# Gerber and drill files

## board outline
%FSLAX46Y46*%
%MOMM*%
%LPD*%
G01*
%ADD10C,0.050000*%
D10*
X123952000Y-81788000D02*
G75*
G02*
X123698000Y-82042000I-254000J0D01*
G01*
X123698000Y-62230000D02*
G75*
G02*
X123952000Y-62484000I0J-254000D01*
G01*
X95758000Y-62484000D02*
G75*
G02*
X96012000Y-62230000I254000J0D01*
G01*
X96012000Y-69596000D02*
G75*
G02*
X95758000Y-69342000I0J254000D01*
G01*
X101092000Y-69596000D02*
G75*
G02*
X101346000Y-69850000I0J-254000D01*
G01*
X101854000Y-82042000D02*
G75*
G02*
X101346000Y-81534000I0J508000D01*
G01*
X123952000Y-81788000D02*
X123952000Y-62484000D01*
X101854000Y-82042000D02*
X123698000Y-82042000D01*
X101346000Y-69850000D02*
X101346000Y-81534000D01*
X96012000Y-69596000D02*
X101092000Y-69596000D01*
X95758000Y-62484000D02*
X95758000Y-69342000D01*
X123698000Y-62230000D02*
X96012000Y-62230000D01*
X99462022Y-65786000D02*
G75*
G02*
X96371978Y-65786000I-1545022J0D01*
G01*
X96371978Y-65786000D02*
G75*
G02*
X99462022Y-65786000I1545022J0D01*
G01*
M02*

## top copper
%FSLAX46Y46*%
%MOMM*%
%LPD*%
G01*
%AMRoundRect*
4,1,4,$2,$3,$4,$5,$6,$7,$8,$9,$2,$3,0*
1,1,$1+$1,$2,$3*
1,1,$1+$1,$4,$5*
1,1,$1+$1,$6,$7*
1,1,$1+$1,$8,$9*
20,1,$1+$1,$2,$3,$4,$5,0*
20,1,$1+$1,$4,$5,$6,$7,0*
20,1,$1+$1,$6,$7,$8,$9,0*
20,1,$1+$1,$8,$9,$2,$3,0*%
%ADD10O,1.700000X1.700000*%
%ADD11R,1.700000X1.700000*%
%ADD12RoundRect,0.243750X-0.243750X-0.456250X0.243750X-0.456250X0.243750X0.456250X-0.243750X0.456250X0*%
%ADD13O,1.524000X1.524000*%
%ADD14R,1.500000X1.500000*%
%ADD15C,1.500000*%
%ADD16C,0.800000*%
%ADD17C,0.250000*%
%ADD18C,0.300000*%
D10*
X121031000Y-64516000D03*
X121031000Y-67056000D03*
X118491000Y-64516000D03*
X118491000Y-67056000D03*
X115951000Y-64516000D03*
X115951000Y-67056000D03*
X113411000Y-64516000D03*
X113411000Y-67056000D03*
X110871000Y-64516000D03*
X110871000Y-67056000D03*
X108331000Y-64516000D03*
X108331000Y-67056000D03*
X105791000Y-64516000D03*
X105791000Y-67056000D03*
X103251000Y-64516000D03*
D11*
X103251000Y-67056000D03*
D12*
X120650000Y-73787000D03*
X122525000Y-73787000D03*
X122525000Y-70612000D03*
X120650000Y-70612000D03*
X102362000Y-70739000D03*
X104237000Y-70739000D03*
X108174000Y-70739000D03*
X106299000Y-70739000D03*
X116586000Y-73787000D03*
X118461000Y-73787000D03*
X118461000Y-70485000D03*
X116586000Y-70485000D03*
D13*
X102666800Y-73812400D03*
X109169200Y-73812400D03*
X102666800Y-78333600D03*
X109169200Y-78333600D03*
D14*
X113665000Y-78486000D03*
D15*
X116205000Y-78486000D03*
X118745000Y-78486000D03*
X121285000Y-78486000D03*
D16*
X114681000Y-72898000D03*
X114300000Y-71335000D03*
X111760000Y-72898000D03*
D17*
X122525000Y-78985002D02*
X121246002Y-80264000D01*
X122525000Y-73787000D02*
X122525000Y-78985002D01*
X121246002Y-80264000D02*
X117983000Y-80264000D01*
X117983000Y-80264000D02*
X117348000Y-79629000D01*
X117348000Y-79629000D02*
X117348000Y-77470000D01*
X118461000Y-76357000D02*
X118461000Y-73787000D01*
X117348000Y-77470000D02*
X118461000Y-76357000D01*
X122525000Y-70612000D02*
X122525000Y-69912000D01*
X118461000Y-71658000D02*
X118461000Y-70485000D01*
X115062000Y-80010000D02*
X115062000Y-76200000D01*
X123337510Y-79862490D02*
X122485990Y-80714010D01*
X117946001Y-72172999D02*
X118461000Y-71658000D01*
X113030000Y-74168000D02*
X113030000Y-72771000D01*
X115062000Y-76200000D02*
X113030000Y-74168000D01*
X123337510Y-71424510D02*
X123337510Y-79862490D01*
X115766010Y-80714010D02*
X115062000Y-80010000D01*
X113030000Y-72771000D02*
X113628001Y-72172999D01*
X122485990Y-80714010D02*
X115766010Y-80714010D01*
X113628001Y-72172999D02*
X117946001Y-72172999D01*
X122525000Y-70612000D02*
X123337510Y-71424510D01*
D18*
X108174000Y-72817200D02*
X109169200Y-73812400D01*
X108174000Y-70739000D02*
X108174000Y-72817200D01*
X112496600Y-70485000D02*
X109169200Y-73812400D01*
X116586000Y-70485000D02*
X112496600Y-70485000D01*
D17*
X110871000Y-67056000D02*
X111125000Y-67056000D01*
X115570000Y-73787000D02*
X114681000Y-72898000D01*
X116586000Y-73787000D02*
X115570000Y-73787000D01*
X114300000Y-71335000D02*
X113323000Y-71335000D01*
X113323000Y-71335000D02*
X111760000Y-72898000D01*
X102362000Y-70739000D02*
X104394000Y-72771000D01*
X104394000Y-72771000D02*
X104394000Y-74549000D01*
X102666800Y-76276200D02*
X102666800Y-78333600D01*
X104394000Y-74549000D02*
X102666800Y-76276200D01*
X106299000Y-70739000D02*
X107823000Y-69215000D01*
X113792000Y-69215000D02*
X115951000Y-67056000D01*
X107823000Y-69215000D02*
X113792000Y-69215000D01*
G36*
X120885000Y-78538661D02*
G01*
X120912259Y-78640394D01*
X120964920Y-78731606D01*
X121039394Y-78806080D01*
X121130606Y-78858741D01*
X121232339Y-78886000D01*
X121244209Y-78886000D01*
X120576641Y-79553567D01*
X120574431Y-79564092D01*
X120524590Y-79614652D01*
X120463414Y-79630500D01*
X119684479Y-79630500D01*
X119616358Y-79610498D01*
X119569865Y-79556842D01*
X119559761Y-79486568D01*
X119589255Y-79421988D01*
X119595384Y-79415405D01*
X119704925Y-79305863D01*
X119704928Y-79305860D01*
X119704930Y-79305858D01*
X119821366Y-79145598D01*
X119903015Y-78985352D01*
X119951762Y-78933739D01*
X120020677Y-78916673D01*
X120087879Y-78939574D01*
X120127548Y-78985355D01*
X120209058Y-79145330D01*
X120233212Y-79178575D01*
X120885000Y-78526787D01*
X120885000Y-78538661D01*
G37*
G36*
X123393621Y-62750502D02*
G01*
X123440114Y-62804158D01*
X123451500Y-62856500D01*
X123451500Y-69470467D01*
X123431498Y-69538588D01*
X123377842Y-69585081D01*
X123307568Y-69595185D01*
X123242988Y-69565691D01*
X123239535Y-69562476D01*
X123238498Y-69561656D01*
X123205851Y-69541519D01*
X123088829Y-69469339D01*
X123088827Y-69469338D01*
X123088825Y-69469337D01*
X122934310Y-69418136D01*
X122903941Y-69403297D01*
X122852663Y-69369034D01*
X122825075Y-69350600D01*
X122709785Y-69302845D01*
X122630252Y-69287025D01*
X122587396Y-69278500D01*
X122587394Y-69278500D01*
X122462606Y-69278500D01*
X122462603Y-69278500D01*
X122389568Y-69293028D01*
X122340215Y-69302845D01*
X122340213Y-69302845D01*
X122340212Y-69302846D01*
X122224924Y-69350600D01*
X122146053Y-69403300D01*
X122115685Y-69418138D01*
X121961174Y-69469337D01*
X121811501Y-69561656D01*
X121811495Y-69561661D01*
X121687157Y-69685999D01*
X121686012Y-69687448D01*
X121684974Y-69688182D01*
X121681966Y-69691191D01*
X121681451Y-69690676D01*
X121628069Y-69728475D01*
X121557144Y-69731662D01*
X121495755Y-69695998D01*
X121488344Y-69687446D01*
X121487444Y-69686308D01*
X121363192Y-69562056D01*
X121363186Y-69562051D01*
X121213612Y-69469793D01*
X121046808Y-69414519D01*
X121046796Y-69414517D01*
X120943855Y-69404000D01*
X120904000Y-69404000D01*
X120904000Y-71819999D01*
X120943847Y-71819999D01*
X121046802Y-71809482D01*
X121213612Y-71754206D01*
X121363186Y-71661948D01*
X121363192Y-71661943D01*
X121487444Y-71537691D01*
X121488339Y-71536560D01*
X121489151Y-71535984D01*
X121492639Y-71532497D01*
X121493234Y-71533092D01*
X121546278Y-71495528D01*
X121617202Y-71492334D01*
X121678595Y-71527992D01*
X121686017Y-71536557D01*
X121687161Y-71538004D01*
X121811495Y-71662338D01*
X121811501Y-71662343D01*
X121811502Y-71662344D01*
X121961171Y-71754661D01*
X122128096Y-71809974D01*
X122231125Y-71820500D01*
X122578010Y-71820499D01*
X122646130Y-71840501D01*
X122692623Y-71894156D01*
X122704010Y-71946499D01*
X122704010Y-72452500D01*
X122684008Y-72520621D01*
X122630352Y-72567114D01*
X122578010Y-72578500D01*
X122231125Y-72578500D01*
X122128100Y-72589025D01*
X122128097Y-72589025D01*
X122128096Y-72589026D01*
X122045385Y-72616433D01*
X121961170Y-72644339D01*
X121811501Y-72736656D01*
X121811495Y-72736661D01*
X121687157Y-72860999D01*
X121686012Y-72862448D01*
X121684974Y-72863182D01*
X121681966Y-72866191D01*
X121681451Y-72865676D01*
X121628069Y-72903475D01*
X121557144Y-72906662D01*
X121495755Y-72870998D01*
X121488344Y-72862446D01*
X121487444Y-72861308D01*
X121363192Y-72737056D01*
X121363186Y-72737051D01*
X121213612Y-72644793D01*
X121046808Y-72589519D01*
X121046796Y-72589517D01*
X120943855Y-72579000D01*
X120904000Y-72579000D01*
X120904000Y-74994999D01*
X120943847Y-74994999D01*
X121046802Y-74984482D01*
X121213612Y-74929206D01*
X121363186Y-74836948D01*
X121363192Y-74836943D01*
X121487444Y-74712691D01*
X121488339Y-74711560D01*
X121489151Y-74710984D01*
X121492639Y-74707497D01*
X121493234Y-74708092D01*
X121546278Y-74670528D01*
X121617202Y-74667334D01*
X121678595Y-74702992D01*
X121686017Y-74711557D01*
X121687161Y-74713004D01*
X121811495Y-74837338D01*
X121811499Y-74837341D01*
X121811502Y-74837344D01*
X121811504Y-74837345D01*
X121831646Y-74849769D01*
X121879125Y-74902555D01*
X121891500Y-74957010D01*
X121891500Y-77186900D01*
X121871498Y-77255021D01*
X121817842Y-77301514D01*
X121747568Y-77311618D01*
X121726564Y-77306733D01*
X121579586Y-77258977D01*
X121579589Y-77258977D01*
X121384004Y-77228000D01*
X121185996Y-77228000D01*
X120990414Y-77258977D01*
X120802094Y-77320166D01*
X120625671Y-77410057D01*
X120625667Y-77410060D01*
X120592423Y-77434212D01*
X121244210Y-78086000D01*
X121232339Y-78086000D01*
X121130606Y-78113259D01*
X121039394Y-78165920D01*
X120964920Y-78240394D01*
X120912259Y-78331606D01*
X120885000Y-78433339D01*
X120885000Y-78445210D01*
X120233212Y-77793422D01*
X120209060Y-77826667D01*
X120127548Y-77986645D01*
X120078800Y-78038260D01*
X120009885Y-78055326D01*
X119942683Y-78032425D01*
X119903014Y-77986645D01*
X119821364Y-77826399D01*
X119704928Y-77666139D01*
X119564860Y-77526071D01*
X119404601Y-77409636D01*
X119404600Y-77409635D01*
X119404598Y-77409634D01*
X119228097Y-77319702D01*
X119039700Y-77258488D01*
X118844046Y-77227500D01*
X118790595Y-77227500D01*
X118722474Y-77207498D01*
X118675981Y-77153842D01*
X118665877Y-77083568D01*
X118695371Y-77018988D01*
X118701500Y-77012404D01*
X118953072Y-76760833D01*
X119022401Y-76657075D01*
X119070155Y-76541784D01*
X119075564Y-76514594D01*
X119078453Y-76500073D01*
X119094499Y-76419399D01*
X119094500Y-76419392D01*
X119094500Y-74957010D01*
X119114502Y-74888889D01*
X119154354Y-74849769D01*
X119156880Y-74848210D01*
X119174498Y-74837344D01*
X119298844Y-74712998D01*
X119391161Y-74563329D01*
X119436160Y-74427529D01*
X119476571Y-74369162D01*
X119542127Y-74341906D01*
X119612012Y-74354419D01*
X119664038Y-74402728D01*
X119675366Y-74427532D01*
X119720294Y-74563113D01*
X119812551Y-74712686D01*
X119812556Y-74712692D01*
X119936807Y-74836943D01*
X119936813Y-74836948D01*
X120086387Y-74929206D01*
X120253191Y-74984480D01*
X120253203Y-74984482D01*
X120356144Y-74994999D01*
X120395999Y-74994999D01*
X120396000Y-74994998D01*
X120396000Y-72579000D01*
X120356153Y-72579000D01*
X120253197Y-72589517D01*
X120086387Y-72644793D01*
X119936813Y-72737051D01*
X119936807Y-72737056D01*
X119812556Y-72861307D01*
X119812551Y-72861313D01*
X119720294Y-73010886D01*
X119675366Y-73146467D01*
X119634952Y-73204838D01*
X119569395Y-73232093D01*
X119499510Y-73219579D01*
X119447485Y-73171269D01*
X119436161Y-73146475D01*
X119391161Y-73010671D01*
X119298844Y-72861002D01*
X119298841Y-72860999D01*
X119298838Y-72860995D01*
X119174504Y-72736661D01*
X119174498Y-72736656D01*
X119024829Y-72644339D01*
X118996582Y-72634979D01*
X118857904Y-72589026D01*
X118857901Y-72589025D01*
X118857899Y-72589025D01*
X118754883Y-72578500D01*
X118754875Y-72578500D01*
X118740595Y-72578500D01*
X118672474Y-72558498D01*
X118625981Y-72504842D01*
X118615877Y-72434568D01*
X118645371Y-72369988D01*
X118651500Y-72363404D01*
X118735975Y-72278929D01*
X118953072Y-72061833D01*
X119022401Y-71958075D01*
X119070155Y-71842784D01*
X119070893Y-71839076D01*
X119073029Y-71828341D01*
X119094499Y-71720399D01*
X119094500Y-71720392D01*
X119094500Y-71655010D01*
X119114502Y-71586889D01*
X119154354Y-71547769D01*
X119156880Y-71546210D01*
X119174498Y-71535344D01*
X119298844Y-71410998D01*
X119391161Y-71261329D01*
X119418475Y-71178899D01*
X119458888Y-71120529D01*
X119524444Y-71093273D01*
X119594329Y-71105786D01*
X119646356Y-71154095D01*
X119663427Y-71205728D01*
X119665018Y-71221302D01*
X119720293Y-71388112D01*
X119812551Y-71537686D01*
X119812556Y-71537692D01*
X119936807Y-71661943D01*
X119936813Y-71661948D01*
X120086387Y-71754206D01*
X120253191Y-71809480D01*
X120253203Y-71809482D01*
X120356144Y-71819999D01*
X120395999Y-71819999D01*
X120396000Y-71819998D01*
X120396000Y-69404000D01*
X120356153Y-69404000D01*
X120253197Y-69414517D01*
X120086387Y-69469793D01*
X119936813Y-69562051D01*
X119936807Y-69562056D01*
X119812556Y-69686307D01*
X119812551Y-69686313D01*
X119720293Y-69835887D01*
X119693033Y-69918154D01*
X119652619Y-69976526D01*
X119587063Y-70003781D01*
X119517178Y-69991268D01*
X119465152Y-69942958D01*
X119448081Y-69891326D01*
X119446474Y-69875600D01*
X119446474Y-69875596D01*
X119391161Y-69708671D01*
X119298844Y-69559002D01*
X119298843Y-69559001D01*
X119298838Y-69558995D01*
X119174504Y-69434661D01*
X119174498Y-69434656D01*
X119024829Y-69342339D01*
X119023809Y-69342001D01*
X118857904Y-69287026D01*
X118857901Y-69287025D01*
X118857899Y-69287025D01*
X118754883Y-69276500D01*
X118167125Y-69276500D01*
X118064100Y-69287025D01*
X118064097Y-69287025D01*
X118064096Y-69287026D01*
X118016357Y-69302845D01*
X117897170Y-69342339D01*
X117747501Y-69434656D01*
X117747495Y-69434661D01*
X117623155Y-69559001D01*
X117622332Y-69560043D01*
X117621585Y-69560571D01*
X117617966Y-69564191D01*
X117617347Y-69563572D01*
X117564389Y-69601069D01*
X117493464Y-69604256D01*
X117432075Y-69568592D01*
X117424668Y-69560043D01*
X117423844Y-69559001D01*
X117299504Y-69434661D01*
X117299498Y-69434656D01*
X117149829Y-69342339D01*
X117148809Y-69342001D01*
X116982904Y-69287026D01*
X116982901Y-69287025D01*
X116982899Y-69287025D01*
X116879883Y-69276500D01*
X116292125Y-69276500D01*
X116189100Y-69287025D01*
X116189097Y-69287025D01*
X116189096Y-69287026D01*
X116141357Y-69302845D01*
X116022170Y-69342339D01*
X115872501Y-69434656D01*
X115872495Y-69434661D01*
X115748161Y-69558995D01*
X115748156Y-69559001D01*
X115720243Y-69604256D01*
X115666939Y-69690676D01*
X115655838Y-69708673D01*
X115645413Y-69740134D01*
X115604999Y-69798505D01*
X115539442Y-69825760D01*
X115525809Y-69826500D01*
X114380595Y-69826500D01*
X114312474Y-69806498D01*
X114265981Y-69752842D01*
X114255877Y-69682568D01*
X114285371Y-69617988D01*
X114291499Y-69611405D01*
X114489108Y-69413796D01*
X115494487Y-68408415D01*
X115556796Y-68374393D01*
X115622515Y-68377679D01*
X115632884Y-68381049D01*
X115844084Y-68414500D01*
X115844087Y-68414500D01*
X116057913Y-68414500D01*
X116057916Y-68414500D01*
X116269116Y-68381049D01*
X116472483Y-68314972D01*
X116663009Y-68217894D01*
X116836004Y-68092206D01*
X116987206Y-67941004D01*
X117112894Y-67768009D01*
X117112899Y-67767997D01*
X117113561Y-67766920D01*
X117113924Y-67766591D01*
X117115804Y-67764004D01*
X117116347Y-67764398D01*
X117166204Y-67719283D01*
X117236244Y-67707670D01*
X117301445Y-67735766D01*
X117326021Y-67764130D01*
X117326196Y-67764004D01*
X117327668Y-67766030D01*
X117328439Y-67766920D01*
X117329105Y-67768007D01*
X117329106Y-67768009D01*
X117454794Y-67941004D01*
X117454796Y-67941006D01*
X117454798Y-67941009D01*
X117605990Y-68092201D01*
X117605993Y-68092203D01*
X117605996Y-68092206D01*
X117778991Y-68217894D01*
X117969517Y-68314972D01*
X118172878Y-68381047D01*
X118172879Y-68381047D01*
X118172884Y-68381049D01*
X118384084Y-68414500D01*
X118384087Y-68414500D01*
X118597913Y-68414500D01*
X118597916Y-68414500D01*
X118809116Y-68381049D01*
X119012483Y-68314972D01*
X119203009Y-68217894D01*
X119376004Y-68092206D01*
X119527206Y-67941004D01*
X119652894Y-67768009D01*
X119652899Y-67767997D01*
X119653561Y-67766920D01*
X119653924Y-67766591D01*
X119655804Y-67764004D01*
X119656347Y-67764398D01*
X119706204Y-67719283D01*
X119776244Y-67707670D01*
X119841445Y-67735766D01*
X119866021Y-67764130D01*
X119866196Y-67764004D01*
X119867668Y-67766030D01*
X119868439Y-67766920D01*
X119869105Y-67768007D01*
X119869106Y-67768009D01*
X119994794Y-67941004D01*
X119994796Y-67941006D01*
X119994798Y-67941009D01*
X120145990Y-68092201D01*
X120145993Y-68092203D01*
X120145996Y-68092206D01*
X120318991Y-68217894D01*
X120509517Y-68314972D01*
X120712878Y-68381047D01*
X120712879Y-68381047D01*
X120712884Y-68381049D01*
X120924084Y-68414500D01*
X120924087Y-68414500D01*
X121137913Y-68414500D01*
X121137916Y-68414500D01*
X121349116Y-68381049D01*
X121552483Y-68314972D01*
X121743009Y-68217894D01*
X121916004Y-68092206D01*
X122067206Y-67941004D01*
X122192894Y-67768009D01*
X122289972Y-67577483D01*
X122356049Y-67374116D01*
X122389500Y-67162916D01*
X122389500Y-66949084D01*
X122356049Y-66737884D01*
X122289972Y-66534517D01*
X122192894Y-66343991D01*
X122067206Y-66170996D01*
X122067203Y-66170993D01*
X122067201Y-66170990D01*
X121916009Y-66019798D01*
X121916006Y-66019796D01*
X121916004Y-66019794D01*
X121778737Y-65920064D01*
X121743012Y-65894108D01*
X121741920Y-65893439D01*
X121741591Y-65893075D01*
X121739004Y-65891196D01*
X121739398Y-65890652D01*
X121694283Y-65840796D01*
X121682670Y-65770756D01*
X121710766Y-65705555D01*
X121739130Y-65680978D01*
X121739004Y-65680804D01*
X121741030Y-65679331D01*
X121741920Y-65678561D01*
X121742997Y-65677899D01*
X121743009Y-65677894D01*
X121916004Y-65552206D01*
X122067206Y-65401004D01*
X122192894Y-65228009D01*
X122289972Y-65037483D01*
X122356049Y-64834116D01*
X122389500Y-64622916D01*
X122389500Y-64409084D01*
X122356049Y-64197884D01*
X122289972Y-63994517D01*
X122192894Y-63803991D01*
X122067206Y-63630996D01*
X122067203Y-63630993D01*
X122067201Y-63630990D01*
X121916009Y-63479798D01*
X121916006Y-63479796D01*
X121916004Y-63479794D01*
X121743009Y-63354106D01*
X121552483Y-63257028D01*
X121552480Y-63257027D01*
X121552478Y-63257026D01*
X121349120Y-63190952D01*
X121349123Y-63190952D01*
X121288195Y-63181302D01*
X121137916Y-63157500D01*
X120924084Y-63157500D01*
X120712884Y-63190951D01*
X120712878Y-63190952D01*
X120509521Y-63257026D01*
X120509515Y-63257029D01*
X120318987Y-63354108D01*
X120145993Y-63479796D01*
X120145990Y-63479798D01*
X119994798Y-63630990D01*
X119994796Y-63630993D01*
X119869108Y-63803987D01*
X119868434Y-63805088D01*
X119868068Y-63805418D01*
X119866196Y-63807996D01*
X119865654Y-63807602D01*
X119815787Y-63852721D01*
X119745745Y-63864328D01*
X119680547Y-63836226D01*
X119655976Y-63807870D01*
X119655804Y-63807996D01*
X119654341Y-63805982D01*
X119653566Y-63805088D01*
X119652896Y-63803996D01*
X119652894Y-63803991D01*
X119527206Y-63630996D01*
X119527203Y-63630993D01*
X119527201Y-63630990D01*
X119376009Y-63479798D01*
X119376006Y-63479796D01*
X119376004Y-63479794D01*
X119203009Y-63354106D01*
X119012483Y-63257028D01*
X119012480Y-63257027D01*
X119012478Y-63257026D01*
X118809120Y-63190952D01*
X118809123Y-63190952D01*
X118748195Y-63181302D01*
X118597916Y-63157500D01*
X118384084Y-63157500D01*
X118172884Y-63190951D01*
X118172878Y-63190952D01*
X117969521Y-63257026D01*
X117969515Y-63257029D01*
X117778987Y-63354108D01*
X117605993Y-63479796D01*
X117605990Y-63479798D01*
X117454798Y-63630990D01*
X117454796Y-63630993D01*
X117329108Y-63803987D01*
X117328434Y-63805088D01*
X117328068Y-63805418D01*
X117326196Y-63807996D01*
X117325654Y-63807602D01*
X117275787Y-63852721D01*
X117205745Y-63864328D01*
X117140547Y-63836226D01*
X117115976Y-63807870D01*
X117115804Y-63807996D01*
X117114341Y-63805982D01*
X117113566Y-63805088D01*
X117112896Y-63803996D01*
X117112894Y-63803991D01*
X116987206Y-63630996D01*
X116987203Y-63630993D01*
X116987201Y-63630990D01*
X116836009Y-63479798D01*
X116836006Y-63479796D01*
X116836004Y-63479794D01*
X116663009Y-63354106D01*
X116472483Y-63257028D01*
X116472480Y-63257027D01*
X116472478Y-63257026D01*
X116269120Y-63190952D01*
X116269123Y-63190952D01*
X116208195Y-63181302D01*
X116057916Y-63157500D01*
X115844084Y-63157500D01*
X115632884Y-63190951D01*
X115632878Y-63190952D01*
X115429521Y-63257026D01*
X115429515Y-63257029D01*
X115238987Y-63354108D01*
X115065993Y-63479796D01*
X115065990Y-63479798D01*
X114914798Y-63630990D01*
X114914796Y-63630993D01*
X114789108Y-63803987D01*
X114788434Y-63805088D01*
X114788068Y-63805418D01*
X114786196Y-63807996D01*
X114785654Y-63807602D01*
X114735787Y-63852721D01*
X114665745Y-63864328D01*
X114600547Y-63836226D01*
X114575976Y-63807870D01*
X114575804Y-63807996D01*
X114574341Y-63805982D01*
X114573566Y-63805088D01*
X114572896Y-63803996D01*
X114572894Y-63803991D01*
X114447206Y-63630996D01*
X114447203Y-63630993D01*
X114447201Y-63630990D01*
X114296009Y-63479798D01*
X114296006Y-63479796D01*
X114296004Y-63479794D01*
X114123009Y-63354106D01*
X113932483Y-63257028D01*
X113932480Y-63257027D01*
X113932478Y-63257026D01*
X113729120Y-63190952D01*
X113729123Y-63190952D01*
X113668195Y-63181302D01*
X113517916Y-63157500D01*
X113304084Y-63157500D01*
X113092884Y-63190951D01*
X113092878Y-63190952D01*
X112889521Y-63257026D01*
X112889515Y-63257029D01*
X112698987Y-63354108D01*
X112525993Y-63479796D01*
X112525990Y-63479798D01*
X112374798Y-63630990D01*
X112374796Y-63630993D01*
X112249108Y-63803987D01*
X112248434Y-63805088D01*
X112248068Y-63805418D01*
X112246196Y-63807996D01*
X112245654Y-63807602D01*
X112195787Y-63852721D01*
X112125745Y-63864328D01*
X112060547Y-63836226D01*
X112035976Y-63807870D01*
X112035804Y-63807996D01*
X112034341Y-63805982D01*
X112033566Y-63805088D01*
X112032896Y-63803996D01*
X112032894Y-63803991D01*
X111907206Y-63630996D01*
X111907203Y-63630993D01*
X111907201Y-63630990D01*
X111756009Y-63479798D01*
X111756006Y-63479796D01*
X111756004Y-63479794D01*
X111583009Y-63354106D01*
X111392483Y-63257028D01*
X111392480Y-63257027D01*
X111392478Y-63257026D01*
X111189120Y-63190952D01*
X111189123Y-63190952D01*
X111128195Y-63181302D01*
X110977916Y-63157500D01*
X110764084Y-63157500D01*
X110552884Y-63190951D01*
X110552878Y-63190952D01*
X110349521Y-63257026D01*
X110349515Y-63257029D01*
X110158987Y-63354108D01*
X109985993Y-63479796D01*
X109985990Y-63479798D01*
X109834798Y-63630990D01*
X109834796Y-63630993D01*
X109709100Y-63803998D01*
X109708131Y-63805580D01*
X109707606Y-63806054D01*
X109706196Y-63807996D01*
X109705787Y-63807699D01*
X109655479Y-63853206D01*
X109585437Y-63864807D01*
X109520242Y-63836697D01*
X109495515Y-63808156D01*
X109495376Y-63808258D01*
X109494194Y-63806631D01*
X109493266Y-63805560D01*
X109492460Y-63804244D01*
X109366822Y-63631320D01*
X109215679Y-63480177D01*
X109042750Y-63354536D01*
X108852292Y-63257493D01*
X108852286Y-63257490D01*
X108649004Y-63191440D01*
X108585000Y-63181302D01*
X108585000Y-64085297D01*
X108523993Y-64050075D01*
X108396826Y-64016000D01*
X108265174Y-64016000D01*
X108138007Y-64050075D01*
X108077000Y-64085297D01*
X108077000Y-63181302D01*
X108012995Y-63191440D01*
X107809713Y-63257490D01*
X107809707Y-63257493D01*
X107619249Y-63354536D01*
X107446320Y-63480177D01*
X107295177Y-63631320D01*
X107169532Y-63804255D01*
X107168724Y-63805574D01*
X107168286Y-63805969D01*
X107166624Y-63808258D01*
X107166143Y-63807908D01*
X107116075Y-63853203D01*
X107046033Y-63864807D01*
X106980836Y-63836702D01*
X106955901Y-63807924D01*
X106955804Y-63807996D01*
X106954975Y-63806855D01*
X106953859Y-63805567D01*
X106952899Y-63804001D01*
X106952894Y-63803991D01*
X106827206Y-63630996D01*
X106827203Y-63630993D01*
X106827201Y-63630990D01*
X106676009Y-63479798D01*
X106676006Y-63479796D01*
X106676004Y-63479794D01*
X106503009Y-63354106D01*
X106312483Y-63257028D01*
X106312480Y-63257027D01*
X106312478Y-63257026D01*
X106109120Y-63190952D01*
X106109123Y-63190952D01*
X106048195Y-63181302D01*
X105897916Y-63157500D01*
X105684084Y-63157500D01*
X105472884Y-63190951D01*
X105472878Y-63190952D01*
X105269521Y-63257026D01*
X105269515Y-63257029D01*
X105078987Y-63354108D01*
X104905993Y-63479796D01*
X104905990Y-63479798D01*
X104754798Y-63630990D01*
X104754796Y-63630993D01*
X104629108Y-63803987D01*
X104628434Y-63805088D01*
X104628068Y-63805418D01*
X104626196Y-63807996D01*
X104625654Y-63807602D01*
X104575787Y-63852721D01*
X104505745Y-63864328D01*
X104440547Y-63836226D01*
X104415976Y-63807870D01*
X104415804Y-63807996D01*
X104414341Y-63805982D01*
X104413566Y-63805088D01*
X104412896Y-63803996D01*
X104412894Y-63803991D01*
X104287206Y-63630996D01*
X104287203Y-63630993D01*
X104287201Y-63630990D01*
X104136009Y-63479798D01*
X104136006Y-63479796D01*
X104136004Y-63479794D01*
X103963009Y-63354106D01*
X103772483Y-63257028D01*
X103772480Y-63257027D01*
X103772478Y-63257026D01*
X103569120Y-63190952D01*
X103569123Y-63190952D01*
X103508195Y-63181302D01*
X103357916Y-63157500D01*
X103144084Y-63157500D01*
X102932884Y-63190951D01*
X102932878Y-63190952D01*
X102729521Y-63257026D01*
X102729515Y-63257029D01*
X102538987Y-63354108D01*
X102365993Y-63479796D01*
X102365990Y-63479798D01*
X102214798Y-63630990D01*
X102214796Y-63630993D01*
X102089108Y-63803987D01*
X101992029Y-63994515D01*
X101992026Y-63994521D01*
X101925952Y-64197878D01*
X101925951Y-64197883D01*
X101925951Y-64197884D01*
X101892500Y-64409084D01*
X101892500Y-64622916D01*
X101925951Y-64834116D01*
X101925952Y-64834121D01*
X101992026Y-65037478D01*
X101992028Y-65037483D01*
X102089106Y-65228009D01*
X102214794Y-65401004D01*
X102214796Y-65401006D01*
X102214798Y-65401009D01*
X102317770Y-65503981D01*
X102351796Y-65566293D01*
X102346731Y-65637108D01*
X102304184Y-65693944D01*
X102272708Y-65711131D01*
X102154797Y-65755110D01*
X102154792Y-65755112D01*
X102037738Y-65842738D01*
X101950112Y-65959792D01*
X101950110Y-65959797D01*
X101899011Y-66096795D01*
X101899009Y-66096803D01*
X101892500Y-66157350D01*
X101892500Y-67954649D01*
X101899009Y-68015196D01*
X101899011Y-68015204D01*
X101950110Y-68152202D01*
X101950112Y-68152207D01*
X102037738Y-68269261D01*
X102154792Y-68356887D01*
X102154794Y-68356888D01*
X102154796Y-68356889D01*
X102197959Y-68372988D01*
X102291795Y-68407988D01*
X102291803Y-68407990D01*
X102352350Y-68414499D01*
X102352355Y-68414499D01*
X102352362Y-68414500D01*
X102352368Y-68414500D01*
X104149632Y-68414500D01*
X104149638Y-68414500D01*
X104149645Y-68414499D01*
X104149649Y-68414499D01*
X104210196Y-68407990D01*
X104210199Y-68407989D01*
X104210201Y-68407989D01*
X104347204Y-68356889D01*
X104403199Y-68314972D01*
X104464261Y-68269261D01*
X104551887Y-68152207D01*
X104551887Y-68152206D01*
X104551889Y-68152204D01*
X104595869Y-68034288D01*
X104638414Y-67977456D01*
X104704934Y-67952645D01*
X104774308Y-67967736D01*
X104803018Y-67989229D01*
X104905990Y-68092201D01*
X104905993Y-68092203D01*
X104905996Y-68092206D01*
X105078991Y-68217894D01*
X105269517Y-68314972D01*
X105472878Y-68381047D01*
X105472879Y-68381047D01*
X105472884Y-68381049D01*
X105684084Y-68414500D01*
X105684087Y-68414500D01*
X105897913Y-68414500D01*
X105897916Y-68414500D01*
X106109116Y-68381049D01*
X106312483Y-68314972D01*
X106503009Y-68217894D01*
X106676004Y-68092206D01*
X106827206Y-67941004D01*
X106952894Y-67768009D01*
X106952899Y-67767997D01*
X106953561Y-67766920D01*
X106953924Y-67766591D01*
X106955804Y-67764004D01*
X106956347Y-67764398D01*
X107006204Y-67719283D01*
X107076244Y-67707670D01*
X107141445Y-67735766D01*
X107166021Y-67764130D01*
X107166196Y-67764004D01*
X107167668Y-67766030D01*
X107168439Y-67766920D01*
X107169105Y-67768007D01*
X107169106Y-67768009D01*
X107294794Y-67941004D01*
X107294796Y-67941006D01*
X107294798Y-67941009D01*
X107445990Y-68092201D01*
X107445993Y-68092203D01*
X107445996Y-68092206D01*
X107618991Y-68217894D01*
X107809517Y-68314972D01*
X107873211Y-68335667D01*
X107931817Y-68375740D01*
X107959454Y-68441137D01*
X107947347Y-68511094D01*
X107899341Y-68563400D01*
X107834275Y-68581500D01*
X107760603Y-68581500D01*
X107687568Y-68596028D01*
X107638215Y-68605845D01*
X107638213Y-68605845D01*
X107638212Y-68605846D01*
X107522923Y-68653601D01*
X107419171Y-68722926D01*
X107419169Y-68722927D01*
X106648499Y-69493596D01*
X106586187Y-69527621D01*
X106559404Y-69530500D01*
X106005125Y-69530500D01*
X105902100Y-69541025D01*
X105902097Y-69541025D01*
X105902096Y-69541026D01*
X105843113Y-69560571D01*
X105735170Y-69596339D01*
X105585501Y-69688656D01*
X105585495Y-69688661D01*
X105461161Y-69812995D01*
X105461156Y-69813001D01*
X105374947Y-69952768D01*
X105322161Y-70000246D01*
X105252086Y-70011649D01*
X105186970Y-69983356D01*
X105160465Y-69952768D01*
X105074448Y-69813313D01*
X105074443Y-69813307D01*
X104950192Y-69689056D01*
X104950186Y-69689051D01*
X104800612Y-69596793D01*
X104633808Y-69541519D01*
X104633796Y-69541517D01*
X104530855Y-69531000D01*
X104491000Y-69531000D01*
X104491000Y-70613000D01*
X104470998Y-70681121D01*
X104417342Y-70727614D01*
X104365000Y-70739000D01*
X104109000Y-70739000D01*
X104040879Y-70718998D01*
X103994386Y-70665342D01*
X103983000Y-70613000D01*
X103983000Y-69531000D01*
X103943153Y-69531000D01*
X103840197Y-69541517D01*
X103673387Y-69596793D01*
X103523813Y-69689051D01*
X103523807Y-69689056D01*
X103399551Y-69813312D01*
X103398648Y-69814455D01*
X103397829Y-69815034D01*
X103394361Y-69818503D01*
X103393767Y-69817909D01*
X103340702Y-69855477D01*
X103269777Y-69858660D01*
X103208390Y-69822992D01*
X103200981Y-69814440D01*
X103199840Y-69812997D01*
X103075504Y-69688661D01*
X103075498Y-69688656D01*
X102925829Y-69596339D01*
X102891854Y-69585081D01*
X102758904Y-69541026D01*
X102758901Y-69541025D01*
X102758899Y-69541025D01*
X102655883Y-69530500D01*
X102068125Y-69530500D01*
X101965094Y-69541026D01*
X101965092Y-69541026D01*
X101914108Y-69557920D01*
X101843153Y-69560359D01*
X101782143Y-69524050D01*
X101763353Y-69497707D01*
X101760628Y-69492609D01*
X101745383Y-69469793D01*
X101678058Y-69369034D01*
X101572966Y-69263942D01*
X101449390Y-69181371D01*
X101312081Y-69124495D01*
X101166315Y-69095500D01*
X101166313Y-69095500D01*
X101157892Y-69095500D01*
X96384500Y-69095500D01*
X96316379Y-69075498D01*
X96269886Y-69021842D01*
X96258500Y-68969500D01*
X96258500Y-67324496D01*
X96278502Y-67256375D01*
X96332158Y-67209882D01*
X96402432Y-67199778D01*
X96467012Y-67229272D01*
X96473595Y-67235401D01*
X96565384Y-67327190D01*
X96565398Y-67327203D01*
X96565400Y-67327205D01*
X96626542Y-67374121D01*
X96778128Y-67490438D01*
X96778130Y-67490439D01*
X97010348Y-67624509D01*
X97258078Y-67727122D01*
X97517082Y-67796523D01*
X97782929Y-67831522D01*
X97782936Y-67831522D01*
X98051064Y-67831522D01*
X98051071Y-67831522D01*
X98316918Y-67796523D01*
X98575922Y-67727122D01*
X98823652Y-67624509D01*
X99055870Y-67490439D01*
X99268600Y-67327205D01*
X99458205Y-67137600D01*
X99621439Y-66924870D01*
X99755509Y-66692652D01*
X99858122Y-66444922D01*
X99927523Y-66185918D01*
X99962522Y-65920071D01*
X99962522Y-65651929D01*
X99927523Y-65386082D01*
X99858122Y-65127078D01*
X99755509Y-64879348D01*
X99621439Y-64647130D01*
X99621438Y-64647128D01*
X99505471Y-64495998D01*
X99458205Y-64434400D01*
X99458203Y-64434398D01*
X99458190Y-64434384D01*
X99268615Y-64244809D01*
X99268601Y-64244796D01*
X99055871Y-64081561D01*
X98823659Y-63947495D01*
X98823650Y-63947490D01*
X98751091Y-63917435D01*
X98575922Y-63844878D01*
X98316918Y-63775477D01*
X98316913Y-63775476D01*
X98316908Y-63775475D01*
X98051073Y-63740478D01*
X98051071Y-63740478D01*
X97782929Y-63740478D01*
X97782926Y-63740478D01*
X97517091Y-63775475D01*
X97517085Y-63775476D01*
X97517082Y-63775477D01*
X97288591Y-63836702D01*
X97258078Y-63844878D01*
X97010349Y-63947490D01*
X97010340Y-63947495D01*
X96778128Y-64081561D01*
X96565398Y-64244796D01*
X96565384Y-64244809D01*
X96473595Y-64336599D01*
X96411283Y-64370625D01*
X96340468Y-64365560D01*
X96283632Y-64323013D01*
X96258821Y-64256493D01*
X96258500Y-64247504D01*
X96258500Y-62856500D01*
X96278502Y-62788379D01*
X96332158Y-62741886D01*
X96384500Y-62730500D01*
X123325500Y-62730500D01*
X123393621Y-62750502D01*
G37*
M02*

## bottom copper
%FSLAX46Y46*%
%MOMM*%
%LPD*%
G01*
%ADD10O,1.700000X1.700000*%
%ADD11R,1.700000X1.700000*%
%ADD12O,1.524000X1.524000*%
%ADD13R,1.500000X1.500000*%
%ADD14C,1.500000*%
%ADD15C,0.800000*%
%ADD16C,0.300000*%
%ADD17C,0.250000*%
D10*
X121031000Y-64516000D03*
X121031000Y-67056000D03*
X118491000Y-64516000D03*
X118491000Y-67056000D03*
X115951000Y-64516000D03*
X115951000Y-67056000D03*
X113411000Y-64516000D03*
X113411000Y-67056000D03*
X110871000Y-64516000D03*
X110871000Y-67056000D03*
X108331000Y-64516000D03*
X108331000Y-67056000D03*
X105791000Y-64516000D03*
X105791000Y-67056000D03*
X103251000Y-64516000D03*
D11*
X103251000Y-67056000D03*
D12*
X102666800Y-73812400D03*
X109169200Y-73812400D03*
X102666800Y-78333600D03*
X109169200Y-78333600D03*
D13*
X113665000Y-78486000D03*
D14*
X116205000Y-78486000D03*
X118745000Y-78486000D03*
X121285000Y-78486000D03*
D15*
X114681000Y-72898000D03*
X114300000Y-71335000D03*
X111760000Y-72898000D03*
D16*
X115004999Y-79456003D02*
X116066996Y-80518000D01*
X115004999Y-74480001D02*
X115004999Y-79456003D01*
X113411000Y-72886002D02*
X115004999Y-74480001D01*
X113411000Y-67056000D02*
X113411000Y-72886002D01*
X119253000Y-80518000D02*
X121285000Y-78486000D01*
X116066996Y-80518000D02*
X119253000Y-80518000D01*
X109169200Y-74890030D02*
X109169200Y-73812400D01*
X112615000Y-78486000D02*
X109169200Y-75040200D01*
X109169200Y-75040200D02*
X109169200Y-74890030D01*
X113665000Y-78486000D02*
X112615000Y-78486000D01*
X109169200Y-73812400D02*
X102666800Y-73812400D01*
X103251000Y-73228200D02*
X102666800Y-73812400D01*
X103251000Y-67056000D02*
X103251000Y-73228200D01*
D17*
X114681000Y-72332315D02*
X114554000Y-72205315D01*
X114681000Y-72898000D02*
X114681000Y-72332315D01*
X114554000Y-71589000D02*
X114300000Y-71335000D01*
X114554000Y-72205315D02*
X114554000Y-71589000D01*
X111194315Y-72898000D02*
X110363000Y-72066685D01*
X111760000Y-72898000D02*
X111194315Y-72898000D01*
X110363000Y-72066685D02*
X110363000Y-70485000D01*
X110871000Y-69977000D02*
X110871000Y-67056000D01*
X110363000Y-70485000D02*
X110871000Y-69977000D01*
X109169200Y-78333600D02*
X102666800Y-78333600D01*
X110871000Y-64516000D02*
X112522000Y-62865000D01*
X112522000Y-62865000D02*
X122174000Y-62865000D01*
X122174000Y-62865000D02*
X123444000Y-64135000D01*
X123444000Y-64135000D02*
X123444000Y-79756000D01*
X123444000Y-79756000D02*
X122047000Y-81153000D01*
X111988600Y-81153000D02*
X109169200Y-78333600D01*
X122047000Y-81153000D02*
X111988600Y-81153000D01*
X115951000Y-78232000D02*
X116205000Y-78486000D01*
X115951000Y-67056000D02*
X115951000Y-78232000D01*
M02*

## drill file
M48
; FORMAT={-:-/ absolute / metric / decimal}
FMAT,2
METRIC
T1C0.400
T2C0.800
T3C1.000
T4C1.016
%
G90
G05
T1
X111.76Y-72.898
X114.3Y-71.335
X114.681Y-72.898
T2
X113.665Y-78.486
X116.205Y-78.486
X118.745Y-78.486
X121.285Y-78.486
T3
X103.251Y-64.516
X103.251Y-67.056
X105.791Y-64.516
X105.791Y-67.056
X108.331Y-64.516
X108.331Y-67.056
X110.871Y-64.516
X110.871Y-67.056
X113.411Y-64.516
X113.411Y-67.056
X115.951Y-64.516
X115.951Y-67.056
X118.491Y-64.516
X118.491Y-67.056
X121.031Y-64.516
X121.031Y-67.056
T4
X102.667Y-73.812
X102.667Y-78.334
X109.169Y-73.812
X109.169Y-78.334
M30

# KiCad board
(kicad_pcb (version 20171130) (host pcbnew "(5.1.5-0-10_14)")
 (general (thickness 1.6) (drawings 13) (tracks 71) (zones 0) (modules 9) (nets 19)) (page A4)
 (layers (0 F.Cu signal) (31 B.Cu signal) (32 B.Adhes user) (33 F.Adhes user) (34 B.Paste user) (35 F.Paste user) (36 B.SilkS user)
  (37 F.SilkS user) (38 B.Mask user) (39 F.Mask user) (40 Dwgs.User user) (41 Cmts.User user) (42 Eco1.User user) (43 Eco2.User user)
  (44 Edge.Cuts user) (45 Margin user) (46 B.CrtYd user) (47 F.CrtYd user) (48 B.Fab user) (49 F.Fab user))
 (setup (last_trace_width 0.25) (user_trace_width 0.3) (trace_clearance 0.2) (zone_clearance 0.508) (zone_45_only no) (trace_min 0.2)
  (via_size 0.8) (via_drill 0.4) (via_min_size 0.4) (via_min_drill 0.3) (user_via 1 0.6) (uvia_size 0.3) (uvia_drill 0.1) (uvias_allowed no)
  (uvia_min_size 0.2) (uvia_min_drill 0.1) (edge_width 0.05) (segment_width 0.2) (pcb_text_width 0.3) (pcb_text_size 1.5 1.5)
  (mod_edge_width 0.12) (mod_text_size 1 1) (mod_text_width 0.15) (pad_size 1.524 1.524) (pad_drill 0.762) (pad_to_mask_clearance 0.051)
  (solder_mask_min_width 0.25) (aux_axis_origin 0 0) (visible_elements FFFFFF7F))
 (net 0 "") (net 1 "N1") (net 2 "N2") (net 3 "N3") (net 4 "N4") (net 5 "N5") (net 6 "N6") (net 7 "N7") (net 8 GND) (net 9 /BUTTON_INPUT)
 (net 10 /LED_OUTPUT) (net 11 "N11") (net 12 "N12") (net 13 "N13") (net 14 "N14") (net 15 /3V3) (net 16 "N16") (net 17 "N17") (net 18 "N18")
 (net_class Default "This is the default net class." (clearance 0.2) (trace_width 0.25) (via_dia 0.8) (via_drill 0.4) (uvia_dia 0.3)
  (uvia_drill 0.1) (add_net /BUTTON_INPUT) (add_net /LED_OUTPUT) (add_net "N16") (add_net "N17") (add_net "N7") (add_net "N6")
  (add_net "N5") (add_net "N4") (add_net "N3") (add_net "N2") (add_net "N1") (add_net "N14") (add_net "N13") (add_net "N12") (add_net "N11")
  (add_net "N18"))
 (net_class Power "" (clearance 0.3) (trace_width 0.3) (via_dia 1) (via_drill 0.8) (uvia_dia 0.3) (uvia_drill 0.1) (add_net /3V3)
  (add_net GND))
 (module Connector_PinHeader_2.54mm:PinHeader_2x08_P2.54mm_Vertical (layer F.Cu) (at 103.251 67.056 90)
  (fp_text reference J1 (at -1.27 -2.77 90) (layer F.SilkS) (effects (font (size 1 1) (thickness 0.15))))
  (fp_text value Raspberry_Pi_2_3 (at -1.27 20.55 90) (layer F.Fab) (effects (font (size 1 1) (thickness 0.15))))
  (pad 16 thru_hole oval (at 2.54 17.78 90) (size 1.7 1.7) (drill 1) (layers *.Cu *.Mask) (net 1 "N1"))
  (pad 15 thru_hole oval (at 0 17.78 90) (size 1.7 1.7) (drill 1) (layers *.Cu *.Mask) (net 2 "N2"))
  (pad 14 thru_hole oval (at 2.54 15.24 90) (size 1.7 1.7) (drill 1) (layers *.Cu *.Mask) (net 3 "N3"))
  (pad 13 thru_hole oval (at 0 15.24 90) (size 1.7 1.7) (drill 1) (layers *.Cu *.Mask) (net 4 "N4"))
  (pad 12 thru_hole oval (at 2.54 12.7 90) (size 1.7 1.7) (drill 1) (layers *.Cu *.Mask) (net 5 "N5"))
  (pad 11 thru_hole oval (at 0 12.7 90) (size 1.7 1.7) (drill 1) (layers *.Cu *.Mask) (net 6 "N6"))
  (pad 10 thru_hole oval (at 2.54 10.16 90) (size 1.7 1.7) (drill 1) (layers *.Cu *.Mask) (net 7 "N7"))
  (pad 9 thru_hole oval (at 0 10.16 90) (size 1.7 1.7) (drill 1) (layers *.Cu *.Mask) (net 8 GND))
  (pad 8 thru_hole oval (at 2.54 7.62 90) (size 1.7 1.7) (drill 1) (layers *.Cu *.Mask) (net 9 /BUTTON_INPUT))
  (pad 7 thru_hole oval (at 0 7.62 90) (size 1.7 1.7) (drill 1) (layers *.Cu *.Mask) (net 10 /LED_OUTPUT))
  (pad 6 thru_hole oval (at 2.54 5.08 90) (size 1.7 1.7) (drill 1) (layers *.Cu *.Mask) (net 8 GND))
  (pad 5 thru_hole oval (at 0 5.08 90) (size 1.7 1.7) (drill 1) (layers *.Cu *.Mask) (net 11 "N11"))
  (pad 4 thru_hole oval (at 2.54 2.54 90) (size 1.7 1.7) (drill 1) (layers *.Cu *.Mask) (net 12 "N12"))
  (pad 3 thru_hole oval (at 0 2.54 90) (size 1.7 1.7) (drill 1) (layers *.Cu *.Mask) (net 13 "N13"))
  (pad 2 thru_hole oval (at 2.54 0 90) (size 1.7 1.7) (drill 1) (layers *.Cu *.Mask) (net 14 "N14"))
  (pad 1 thru_hole rect (at 0 0 90) (size 1.7 1.7) (drill 1) (layers *.Cu *.Mask) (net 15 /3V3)))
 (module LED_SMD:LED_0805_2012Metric (layer F.Cu) (at 121.5875 73.787)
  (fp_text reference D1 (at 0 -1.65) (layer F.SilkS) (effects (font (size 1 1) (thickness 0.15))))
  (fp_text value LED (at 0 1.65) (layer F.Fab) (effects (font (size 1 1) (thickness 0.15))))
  (pad 1 smd roundrect (at -0.9375 0) (size 0.975 1.4) (layers F.Cu F.Paste F.Mask) (roundrect_rratio 0.25) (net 8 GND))
  (pad 2 smd roundrect (at 0.9375 0) (size 0.975 1.4) (layers F.Cu F.Paste F.Mask) (roundrect_rratio 0.25) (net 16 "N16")))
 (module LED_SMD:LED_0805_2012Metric (layer F.Cu) (at 121.5875 70.612)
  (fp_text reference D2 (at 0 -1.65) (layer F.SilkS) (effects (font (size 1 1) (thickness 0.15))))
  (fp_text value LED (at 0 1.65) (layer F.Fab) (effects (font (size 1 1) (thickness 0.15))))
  (pad 2 smd roundrect (at 0.9375 0) (size 0.975 1.4) (layers F.Cu F.Paste F.Mask) (roundrect_rratio 0.25) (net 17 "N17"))
  (pad 1 smd roundrect (at -0.9375 0) (size 0.975 1.4) (layers F.Cu F.Paste F.Mask) (roundrect_rratio 0.25) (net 8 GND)))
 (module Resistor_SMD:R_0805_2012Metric (layer F.Cu) (at 103.2995 70.739)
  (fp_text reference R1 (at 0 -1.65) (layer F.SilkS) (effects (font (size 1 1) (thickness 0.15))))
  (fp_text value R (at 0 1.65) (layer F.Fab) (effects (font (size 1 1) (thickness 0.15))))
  (pad 1 smd roundrect (at -0.9375 0) (size 0.975 1.4) (layers F.Cu F.Paste F.Mask) (roundrect_rratio 0.25) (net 9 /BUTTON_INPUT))
  (pad 2 smd roundrect (at 0.9375 0) (size 0.975 1.4) (layers F.Cu F.Paste F.Mask) (roundrect_rratio 0.25) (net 8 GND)))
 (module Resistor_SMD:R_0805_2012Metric (layer F.Cu) (at 107.2365 70.739)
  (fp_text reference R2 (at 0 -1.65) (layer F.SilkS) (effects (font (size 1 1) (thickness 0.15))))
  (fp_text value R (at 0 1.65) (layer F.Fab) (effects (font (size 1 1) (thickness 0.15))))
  (pad 2 smd roundrect (at 0.9375 0) (size 0.975 1.4) (layers F.Cu F.Paste F.Mask) (roundrect_rratio 0.25) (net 15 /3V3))
  (pad 1 smd roundrect (at -0.9375 0) (size 0.975 1.4) (layers F.Cu F.Paste F.Mask) (roundrect_rratio 0.25) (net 6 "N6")))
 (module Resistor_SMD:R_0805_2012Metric (layer F.Cu) (at 117.5235 73.787)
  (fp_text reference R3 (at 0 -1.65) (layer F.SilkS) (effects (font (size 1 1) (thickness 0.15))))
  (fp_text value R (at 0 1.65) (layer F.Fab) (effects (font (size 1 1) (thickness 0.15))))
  (pad 1 smd roundrect (at -0.9375 0) (size 0.975 1.4) (layers F.Cu F.Paste F.Mask) (roundrect_rratio 0.25) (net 10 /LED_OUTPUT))
  (pad 2 smd roundrect (at 0.9375 0) (size 0.975 1.4) (layers F.Cu F.Paste F.Mask) (roundrect_rratio 0.25) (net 16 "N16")))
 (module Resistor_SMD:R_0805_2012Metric (layer F.Cu) (at 117.5235 70.485)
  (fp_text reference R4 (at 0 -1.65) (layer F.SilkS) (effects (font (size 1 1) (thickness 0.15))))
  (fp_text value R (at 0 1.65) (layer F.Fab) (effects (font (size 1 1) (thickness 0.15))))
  (pad 2 smd roundrect (at 0.9375 0) (size 0.975 1.4) (layers F.Cu F.Paste F.Mask) (roundrect_rratio 0.25) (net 17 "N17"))
  (pad 1 smd roundrect (at -0.9375 0) (size 0.975 1.4) (layers F.Cu F.Paste F.Mask) (roundrect_rratio 0.25) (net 15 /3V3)))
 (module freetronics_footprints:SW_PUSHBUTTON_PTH (layer F.Cu) (at 105.918 76.073)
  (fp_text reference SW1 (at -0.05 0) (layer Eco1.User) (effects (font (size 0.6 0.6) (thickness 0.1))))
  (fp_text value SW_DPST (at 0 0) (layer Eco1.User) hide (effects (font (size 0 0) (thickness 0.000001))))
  (pad 1 thru_hole oval (at -3.2512 -2.2606) (size 1.524 1.524) (drill 1.016) (layers *.Cu *.Mask) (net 15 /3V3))
  (pad 1 thru_hole oval (at 3.2512 -2.2606) (size 1.524 1.524) (drill 1.016) (layers *.Cu *.Mask) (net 15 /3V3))
  (pad 2 thru_hole oval (at -3.2512 2.2606) (size 1.524 1.524) (drill 1.016) (layers *.Cu *.Mask) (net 9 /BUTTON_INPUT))
  (pad 2 thru_hole oval (at 3.2512 2.2606) (size 1.524 1.524) (drill 1.016) (layers *.Cu *.Mask) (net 9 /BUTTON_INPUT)))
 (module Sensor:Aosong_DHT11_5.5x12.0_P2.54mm (layer F.Cu) (at 113.665 78.486 90)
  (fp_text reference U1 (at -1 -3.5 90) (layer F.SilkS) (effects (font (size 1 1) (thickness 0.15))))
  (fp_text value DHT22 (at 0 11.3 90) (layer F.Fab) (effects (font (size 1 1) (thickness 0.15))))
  (pad 1 thru_hole rect (at 0 0 90) (size 1.5 1.5) (drill 0.8) (layers *.Cu *.Mask) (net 15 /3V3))
  (pad 2 thru_hole circle (at 0 2.54 90) (size 1.5 1.5) (drill 0.8) (layers *.Cu *.Mask) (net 6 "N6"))
  (pad 3 thru_hole circle (at 0 5.08 90) (size 1.5 1.5) (drill 0.8) (layers *.Cu *.Mask) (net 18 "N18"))
  (pad 4 thru_hole circle (at 0 7.62 90) (size 1.5 1.5) (drill 0.8) (layers *.Cu *.Mask) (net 8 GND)))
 (gr_arc (start 123.698 81.788) (end 123.698 82.042) (angle -90) (layer Edge.Cuts) (width 0.05))
 (gr_arc (start 123.698 62.484) (end 123.952 62.484) (angle -90) (layer Edge.Cuts) (width 0.05))
 (gr_arc (start 96.012 62.484) (end 96.012 62.23) (angle -90) (layer Edge.Cuts) (width 0.05))
 (gr_arc (start 96.012 69.342) (end 95.758 69.342) (angle -90) (layer Edge.Cuts) (width 0.05))
 (gr_arc (start 101.092 69.85) (end 101.346 69.85) (angle -90) (layer Edge.Cuts) (width 0.05))
 (gr_arc (start 101.854 81.534) (end 101.346 81.534) (angle -90) (layer Edge.Cuts) (width 0.05))
 (gr_line (start 123.952 81.788) (end 123.952 62.484) (layer Edge.Cuts) (width 0.05))
 (gr_line (start 101.854 82.042) (end 123.698 82.042) (layer Edge.Cuts) (width 0.05))
 (gr_line (start 101.346 69.85) (end 101.346 81.534) (layer Edge.Cuts) (width 0.05))
 (gr_line (start 96.012 69.596) (end 101.092 69.596) (layer Edge.Cuts) (width 0.05))
 (gr_line (start 95.758 62.484) (end 95.758 69.342) (layer Edge.Cuts) (width 0.05))
 (gr_line (start 123.698 62.23) (end 96.012 62.23) (layer Edge.Cuts) (width 0.05))
 (gr_circle (center 97.917 65.786) (end 99.441 66.04) (layer Edge.Cuts) (width 0.05))
 (segment (start 115.004999 79.456003) (end 116.066996 80.518) (width 0.3) (layer B.Cu) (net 8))
 (segment (start 115.004999 74.480001) (end 115.004999 79.456003) (width 0.3) (layer B.Cu) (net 8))
 (segment (start 113.411 72.886002) (end 115.004999 74.480001) (width 0.3) (layer B.Cu) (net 8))
 (segment (start 113.411 67.056) (end 113.411 72.886002) (width 0.3) (layer B.Cu) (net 8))
 (segment (start 119.253 80.518) (end 121.285 78.486) (width 0.3) (layer B.Cu) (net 8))
 (segment (start 116.066996 80.518) (end 119.253 80.518) (width 0.3) (layer B.Cu) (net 8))
 (segment (start 122.525 78.985002) (end 121.246002 80.264) (width 0.25) (layer F.Cu) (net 16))
 (segment (start 122.525 73.787) (end 122.525 78.985002) (width 0.25) (layer F.Cu) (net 16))
 (segment (start 121.246002 80.264) (end 117.983 80.264) (width 0.25) (layer F.Cu) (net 16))
 (segment (start 117.983 80.264) (end 117.348 79.629) (width 0.25) (layer F.Cu) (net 16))
 (segment (start 117.348 79.629) (end 117.348 77.47) (width 0.25) (layer F.Cu) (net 16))
 (segment (start 118.461 76.357) (end 118.461 73.787) (width 0.25) (layer F.Cu) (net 16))
 (segment (start 117.348 77.47) (end 118.461 76.357) (width 0.25) (layer F.Cu) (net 16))
 (segment (start 122.525 70.612) (end 122.525 69.912) (width 0.25) (layer F.Cu) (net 17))
 (segment (start 118.461 71.658) (end 118.461 70.485) (width 0.25) (layer F.Cu) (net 17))
 (segment (start 115.062 80.01) (end 115.062 76.2) (width 0.25) (layer F.Cu) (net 17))
 (segment (start 123.33751 79.86249) (end 122.48599 80.71401) (width 0.25) (layer F.Cu) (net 17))
 (segment (start 117.946001 72.172999) (end 118.461 71.658) (width 0.25) (layer F.Cu) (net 17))
 (segment (start 113.03 74.168) (end 113.03 72.771) (width 0.25) (layer F.Cu) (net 17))
 (segment (start 115.062 76.2) (end 113.03 74.168) (width 0.25) (layer F.Cu) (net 17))
 (segment (start 123.33751 71.42451) (end 123.33751 79.86249) (width 0.25) (layer F.Cu) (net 17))
 (segment (start 115.76601 80.71401) (end 115.062 80.01) (width 0.25) (layer F.Cu) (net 17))
 (segment (start 113.03 72.771) (end 113.628001 72.172999) (width 0.25) (layer F.Cu) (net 17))
 (segment (start 122.48599 80.71401) (end 115.76601 80.71401) (width 0.25) (layer F.Cu) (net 17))
 (segment (start 113.628001 72.172999) (end 117.946001 72.172999) (width 0.25) (layer F.Cu) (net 17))
 (segment (start 122.525 70.612) (end 123.33751 71.42451) (width 0.25) (layer F.Cu) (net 17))
 (segment (start 109.1692 74.89003) (end 109.1692 73.8124) (width 0.3) (layer B.Cu) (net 15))
 (segment (start 112.615 78.486) (end 109.1692 75.0402) (width 0.3) (layer B.Cu) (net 15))
 (segment (start 109.1692 75.0402) (end 109.1692 74.89003) (width 0.3) (layer B.Cu) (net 15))
 (segment (start 113.665 78.486) (end 112.615 78.486) (width 0.3) (layer B.Cu) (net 15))
 (segment (start 109.1692 73.8124) (end 102.6668 73.8124) (width 0.3) (layer B.Cu) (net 15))
 (segment (start 103.251 73.2282) (end 102.6668 73.8124) (width 0.3) (layer B.Cu) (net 15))
 (segment (start 103.251 67.056) (end 103.251 73.2282) (width 0.3) (layer B.Cu) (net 15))
 (segment (start 108.174 72.8172) (end 109.1692 73.8124) (width 0.3) (layer F.Cu) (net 15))
 (segment (start 108.174 70.739) (end 108.174 72.8172) (width 0.3) (layer F.Cu) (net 15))
 (segment (start 112.4966 70.485) (end 109.1692 73.8124) (width 0.3) (layer F.Cu) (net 15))
 (segment (start 116.586 70.485) (end 112.4966 70.485) (width 0.3) (layer F.Cu) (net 15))
 (segment (start 110.871 67.056) (end 111.125 67.056) (width 0.25) (layer F.Cu) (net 10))
 (via (at 114.681 72.898) (size 0.8) (drill 0.4) (layers F.Cu B.Cu) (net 10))
 (segment (start 115.57 73.787) (end 114.681 72.898) (width 0.25) (layer F.Cu) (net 10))
 (segment (start 116.586 73.787) (end 115.57 73.787) (width 0.25) (layer F.Cu) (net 10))
 (segment (start 114.681 72.332315) (end 114.554 72.205315) (width 0.25) (layer B.Cu) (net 10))
 (segment (start 114.681 72.898) (end 114.681 72.332315) (width 0.25) (layer B.Cu) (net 10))
 (via (at 114.3 71.335) (size 0.8) (drill 0.4) (layers F.Cu B.Cu) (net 10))
 (segment (start 114.554 71.589) (end 114.3 71.335) (width 0.25) (layer B.Cu) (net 10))
 (segment (start 114.554 72.205315) (end 114.554 71.589) (width 0.25) (layer B.Cu) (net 10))
 (segment (start 114.3 71.335) (end 113.323 71.335) (width 0.25) (layer F.Cu) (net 10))
 (segment (start 113.323 71.335) (end 111.76 72.898) (width 0.25) (layer F.Cu) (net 10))
 (via (at 111.76 72.898) (size 0.8) (drill 0.4) (layers F.Cu B.Cu) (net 10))
 (segment (start 111.194315 72.898) (end 110.363 72.066685) (width 0.25) (layer B.Cu) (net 10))
 (segment (start 111.76 72.898) (end 111.194315 72.898) (width 0.25) (layer B.Cu) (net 10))
 (segment (start 110.363 72.066685) (end 110.363 70.485) (width 0.25) (layer B.Cu) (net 10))
 (segment (start 110.871 69.977) (end 110.871 67.056) (width 0.25) (layer B.Cu) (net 10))
 (segment (start 110.363 70.485) (end 110.871 69.977) (width 0.25) (layer B.Cu) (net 10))
 (segment (start 109.1692 78.3336) (end 102.6668 78.3336) (width 0.25) (layer B.Cu) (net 9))
 (segment (start 110.871 64.516) (end 112.522 62.865) (width 0.25) (layer B.Cu) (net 9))
 (segment (start 112.522 62.865) (end 122.174 62.865) (width 0.25) (layer B.Cu) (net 9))
 (segment (start 122.174 62.865) (end 123.444 64.135) (width 0.25) (layer B.Cu) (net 9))
 (segment (start 123.444 64.135) (end 123.444 79.756) (width 0.25) (layer B.Cu) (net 9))
 (segment (start 123.444 79.756) (end 122.047 81.153) (width 0.25) (layer B.Cu) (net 9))
 (segment (start 111.9886 81.153) (end 109.1692 78.3336) (width 0.25) (layer B.Cu) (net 9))
 (segment (start 122.047 81.153) (end 111.9886 81.153) (width 0.25) (layer B.Cu) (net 9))
 (segment (start 102.362 70.739) (end 104.394 72.771) (width 0.25) (layer F.Cu) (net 9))
 (segment (start 104.394 72.771) (end 104.394 74.549) (width 0.25) (layer F.Cu) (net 9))
 (segment (start 102.6668 76.2762) (end 102.6668 78.3336) (width 0.25) (layer F.Cu) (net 9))
 (segment (start 104.394 74.549) (end 102.6668 76.2762) (width 0.25) (layer F.Cu) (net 9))
 (segment (start 115.951 78.232) (end 116.205 78.486) (width 0.25) (layer B.Cu) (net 6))
 (segment (start 115.951 67.056) (end 115.951 78.232) (width 0.25) (layer B.Cu) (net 6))
 (segment (start 106.299 70.739) (end 107.823 69.215) (width 0.25) (layer F.Cu) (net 6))
 (segment (start 113.792 69.215) (end 115.951 67.056) (width 0.25) (layer F.Cu) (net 6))
 (segment (start 107.823 69.215) (end 113.792 69.215) (width 0.25) (layer F.Cu) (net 6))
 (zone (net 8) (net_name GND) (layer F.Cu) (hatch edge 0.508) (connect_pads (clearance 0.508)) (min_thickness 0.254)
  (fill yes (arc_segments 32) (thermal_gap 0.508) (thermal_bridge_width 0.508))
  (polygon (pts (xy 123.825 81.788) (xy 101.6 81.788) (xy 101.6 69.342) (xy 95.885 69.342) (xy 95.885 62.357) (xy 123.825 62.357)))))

